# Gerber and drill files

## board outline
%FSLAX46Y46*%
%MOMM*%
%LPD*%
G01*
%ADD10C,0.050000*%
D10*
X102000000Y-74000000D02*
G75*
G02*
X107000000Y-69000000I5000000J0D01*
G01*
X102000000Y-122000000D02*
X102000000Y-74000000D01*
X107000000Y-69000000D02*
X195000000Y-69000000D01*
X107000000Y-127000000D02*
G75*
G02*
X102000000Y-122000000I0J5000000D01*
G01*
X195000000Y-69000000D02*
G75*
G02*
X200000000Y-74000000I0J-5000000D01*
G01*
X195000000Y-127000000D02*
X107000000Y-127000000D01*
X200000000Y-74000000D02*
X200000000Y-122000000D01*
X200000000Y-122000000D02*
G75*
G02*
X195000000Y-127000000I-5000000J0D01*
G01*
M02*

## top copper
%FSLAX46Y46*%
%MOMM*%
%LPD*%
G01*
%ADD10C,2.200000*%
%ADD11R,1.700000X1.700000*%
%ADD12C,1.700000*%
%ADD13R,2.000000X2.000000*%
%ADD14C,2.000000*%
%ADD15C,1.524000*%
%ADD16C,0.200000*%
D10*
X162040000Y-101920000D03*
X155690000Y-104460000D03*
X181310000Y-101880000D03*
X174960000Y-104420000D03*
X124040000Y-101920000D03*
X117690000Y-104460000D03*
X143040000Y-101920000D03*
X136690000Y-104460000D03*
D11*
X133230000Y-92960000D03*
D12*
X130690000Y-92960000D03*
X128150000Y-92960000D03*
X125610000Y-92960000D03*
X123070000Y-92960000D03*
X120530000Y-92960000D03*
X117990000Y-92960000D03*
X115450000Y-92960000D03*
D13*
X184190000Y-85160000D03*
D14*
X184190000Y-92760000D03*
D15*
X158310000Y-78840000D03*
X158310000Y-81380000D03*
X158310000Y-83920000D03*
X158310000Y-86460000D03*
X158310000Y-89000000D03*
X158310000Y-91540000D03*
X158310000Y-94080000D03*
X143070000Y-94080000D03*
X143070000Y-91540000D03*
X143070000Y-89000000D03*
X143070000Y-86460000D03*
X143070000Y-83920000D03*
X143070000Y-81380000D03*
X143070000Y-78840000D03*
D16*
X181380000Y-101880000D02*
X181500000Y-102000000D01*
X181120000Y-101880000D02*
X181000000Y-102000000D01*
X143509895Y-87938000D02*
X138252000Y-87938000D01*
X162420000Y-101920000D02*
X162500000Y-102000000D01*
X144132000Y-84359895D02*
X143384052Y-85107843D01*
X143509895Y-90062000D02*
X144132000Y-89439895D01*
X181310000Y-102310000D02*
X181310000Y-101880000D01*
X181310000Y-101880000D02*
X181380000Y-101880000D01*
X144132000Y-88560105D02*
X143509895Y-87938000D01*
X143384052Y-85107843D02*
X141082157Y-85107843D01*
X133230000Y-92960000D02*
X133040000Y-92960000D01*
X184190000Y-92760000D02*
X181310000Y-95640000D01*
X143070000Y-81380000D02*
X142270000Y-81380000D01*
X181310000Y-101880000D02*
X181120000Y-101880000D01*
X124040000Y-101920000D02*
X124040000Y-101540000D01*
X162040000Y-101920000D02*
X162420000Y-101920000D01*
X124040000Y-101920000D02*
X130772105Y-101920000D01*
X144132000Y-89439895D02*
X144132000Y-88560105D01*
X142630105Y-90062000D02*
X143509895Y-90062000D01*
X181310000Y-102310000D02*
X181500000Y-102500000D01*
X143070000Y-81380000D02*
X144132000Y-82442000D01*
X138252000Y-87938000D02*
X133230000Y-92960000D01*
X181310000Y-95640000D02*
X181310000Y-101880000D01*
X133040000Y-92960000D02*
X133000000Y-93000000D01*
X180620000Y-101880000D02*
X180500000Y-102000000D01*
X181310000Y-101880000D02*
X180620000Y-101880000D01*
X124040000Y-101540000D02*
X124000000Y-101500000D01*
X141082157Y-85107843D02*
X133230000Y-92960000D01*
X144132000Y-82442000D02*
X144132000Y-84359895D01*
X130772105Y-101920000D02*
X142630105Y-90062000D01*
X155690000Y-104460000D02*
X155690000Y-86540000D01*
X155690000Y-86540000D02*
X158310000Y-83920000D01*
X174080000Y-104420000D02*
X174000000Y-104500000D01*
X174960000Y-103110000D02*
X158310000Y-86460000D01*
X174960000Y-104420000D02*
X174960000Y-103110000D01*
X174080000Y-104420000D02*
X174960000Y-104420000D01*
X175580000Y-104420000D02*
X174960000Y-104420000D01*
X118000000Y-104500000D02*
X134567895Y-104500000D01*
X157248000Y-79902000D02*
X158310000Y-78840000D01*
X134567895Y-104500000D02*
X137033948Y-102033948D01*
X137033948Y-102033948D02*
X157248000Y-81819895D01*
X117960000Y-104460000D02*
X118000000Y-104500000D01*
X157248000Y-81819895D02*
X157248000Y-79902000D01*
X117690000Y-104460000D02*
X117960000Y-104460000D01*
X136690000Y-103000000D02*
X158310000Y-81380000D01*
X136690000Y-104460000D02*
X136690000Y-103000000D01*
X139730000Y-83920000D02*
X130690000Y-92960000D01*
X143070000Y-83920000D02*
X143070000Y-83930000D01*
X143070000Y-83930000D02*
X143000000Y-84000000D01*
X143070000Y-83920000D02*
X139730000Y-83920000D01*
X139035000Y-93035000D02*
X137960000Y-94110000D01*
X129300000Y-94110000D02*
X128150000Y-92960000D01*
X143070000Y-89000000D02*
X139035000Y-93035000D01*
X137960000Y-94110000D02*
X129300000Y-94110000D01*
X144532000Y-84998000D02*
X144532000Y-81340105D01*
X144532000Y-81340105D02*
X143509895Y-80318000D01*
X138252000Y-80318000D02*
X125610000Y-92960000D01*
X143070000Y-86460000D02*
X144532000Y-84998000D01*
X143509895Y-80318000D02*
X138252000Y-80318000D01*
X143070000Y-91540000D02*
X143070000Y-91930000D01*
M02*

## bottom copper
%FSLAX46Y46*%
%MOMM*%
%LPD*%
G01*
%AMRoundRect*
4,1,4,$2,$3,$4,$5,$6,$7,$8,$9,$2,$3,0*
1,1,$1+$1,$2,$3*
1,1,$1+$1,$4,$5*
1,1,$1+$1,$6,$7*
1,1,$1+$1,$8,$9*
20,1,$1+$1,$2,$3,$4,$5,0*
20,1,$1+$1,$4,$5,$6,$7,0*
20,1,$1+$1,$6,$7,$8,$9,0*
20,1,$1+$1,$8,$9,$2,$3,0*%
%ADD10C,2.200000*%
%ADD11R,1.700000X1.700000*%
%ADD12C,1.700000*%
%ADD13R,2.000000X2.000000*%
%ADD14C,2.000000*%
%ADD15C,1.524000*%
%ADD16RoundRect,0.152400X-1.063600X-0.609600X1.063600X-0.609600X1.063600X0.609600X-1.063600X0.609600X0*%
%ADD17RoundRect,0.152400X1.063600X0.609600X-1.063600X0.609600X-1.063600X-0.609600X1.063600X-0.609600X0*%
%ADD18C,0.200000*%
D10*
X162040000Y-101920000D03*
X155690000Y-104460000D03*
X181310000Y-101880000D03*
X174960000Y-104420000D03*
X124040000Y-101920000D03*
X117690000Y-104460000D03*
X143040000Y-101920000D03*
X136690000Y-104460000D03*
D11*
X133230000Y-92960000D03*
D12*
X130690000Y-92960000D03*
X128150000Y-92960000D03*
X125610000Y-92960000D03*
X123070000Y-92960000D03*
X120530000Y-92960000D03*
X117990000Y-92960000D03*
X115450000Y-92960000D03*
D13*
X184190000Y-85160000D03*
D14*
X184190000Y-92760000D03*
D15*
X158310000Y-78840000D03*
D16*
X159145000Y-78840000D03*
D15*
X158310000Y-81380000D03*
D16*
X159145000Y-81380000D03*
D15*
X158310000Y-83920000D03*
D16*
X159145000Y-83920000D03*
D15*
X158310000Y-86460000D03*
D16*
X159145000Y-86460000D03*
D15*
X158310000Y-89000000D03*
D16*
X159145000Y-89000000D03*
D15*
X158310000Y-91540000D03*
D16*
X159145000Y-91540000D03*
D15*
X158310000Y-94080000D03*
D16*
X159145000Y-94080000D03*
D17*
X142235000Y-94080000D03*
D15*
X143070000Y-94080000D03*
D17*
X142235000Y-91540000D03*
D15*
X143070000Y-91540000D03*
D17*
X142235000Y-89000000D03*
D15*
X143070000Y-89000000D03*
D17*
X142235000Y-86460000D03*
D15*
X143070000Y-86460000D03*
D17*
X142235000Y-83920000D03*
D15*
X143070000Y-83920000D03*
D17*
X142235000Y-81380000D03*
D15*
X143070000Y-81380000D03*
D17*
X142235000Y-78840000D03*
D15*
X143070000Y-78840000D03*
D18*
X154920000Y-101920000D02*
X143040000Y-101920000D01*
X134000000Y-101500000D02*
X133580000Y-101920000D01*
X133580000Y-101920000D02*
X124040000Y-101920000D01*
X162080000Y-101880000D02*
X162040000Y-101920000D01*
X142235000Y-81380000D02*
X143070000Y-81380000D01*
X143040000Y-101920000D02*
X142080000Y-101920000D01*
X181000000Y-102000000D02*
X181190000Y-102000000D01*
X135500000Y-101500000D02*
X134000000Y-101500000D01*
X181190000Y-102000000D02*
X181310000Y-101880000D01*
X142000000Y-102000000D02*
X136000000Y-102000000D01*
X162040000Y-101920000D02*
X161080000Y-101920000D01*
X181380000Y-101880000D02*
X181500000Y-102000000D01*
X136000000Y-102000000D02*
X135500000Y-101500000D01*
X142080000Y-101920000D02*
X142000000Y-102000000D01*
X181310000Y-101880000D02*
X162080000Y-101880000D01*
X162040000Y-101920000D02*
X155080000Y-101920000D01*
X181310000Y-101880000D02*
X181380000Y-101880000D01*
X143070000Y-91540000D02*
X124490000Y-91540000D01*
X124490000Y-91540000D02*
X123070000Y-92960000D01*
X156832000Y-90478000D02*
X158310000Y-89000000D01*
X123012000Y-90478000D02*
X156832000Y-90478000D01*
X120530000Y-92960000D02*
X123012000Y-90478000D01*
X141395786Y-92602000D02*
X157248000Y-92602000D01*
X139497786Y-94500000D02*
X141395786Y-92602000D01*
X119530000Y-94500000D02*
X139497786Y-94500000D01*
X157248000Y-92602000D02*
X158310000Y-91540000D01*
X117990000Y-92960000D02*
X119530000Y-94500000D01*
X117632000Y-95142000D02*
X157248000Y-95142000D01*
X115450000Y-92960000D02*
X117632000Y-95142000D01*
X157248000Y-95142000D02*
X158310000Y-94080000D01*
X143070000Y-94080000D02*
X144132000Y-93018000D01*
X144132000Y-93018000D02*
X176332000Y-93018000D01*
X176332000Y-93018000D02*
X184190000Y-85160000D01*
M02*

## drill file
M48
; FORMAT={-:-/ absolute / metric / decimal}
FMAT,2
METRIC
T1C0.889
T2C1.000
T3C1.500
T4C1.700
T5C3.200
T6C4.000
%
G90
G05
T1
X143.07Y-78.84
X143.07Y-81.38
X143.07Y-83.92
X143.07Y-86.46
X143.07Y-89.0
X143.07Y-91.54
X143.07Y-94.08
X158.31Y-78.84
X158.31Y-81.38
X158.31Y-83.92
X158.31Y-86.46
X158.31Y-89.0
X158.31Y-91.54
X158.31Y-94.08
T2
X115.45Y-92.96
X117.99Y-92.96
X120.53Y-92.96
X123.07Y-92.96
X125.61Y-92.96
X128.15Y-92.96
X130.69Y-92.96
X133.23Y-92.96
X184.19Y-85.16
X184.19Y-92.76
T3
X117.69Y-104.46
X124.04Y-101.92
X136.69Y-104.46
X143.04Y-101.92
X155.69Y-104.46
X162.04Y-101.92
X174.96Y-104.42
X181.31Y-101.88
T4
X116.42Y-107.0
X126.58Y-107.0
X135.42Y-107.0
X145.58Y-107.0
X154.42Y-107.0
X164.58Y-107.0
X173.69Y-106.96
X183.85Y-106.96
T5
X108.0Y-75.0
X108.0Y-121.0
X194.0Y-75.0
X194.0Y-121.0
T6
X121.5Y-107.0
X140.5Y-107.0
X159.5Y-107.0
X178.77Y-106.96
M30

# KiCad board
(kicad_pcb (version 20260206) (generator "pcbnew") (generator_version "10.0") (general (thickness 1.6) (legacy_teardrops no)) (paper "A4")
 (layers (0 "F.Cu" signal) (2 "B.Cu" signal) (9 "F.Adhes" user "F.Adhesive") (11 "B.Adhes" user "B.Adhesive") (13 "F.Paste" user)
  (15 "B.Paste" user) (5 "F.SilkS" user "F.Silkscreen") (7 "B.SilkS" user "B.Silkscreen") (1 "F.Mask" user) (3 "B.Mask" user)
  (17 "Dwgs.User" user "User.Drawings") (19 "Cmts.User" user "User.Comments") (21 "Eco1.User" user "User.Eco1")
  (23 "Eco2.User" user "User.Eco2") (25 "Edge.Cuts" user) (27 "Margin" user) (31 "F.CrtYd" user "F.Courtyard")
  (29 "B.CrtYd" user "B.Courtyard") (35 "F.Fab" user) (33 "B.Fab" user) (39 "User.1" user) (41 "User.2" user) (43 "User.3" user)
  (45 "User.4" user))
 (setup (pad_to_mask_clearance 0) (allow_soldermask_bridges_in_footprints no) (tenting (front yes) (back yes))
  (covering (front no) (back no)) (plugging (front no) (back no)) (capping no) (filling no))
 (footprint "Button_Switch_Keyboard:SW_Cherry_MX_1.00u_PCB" (layer "F.Cu") (at 162.04 101.92)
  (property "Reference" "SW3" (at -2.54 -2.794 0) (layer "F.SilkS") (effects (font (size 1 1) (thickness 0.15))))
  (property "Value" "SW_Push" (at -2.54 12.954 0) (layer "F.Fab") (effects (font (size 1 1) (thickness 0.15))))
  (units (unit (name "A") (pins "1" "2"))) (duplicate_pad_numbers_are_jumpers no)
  (pad "" np_thru_hole circle (at -7.62 5.08) (size 1.7 1.7) (drill 1.7) (layers "*.Cu" "*.Mask"))
  (pad "" np_thru_hole circle (at -2.54 5.08) (size 4 4) (drill 4) (layers "*.Cu" "*.Mask"))
  (pad "" np_thru_hole circle (at 2.54 5.08) (size 1.7 1.7) (drill 1.7) (layers "*.Cu" "*.Mask"))
  (pad "1" thru_hole circle (at 0 0) (size 2.2 2.2) (drill 1.5) (layers "*.Cu" "*.Mask") (remove_unused_layers no) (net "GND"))
  (pad "2" thru_hole circle (at -6.35 2.54) (size 2.2 2.2) (drill 1.5) (layers "*.Cu" "*.Mask") (remove_unused_layers no)
   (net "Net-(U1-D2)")))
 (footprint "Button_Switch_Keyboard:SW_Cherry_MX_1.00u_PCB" (layer "F.Cu") (at 181.31 101.88)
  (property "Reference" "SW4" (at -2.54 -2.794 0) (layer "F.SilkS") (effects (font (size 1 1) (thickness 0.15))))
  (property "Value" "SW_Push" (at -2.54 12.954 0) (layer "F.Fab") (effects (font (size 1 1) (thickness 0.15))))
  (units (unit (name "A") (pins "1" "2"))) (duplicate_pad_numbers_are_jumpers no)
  (pad "" np_thru_hole circle (at -7.62 5.08) (size 1.7 1.7) (drill 1.7) (layers "*.Cu" "*.Mask"))
  (pad "" np_thru_hole circle (at -2.54 5.08) (size 4 4) (drill 4) (layers "*.Cu" "*.Mask"))
  (pad "" np_thru_hole circle (at 2.54 5.08) (size 1.7 1.7) (drill 1.7) (layers "*.Cu" "*.Mask"))
  (pad "1" thru_hole circle (at 0 0) (size 2.2 2.2) (drill 1.5) (layers "*.Cu" "*.Mask") (remove_unused_layers no) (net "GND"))
  (pad "2" thru_hole circle (at -6.35 2.54) (size 2.2 2.2) (drill 1.5) (layers "*.Cu" "*.Mask") (remove_unused_layers no)
   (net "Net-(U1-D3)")))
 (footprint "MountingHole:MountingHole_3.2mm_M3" (layer "F.Cu") (at 194 121)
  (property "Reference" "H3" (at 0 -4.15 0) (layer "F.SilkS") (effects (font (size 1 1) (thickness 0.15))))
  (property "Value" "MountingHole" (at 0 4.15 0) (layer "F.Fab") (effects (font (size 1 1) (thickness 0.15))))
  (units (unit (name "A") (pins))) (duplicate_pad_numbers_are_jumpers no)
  (pad "" np_thru_hole circle (at 0 0) (size 3.2 3.2) (drill 3.2) (layers "*.Cu" "*.Mask")))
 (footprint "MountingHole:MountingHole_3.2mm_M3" (layer "F.Cu") (at 108 121)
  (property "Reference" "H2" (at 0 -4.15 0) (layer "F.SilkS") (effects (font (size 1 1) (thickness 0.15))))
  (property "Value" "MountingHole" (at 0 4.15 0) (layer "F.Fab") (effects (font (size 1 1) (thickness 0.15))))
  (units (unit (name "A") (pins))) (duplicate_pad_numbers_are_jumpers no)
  (pad "" np_thru_hole circle (at 0 0) (size 3.2 3.2) (drill 3.2) (layers "*.Cu" "*.Mask")))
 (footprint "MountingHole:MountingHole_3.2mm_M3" (layer "F.Cu") (at 194 75)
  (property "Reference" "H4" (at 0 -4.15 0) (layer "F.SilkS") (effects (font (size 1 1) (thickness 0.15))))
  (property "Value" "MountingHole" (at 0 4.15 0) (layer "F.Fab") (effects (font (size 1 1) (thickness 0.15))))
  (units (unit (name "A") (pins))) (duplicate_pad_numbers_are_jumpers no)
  (pad "" np_thru_hole circle (at 0 0) (size 3.2 3.2) (drill 3.2) (layers "*.Cu" "*.Mask")))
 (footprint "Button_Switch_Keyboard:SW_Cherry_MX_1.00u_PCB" (layer "F.Cu") (at 124.04 101.92)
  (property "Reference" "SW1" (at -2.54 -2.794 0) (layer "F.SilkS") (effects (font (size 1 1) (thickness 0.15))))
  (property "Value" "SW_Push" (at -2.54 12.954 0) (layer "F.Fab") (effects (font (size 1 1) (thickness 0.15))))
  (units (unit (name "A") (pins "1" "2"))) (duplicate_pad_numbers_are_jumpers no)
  (pad "" np_thru_hole circle (at -7.62 5.08) (size 1.7 1.7) (drill 1.7) (layers "*.Cu" "*.Mask"))
  (pad "" np_thru_hole circle (at -2.54 5.08) (size 4 4) (drill 4) (layers "*.Cu" "*.Mask"))
  (pad "" np_thru_hole circle (at 2.54 5.08) (size 1.7 1.7) (drill 1.7) (layers "*.Cu" "*.Mask"))
  (pad "1" thru_hole circle (at 0 0) (size 2.2 2.2) (drill 1.5) (layers "*.Cu" "*.Mask") (remove_unused_layers no) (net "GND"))
  (pad "2" thru_hole circle (at -6.35 2.54) (size 2.2 2.2) (drill 1.5) (layers "*.Cu" "*.Mask") (remove_unused_layers no)
   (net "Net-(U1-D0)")))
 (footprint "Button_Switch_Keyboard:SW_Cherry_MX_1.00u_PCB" (layer "F.Cu") (at 143.04 101.92)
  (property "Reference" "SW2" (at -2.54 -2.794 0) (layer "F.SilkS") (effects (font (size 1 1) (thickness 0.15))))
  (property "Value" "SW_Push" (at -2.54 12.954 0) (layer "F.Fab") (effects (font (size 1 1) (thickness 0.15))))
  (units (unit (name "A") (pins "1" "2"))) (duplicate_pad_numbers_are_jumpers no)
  (pad "" np_thru_hole circle (at -7.62 5.08) (size 1.7 1.7) (drill 1.7) (layers "*.Cu" "*.Mask"))
  (pad "" np_thru_hole circle (at -2.54 5.08) (size 4 4) (drill 4) (layers "*.Cu" "*.Mask"))
  (pad "" np_thru_hole circle (at 2.54 5.08) (size 1.7 1.7) (drill 1.7) (layers "*.Cu" "*.Mask"))
  (pad "1" thru_hole circle (at 0 0) (size 2.2 2.2) (drill 1.5) (layers "*.Cu" "*.Mask") (remove_unused_layers no) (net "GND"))
  (pad "2" thru_hole circle (at -6.35 2.54) (size 2.2 2.2) (drill 1.5) (layers "*.Cu" "*.Mask") (remove_unused_layers no)
   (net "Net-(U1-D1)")))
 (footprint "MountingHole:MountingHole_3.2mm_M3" (layer "F.Cu") (at 108 75)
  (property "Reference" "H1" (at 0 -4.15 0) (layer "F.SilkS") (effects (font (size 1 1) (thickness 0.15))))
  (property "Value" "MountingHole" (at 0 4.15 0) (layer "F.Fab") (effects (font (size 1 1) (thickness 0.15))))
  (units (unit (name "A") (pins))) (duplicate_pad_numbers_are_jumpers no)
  (pad "" np_thru_hole circle (at 0 0) (size 3.2 3.2) (drill 3.2) (layers "*.Cu" "*.Mask")))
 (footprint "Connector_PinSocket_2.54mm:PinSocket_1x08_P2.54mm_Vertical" (layer "B.Cu") (at 133.23 92.96 90)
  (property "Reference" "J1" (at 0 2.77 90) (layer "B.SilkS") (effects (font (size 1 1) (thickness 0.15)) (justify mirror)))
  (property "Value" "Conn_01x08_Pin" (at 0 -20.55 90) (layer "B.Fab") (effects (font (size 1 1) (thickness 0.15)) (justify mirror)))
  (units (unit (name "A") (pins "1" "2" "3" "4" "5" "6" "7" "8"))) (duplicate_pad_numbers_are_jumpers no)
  (pad "1" thru_hole rect (at 0 0 90) (size 1.7 1.7) (drill 1) (layers "*.Cu" "*.Mask") (remove_unused_layers no) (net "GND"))
  (pad "2" thru_hole circle (at 0 -2.54 90) (size 1.7 1.7) (drill 1) (layers "*.Cu" "*.Mask") (remove_unused_layers no) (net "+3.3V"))
  (pad "3" thru_hole circle (at 0 -5.08 90) (size 1.7 1.7) (drill 1) (layers "*.Cu" "*.Mask") (remove_unused_layers no) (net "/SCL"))
  (pad "4" thru_hole circle (at 0 -7.62 90) (size 1.7 1.7) (drill 1) (layers "*.Cu" "*.Mask") (remove_unused_layers no) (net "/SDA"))
  (pad "5" thru_hole circle (at 0 -10.16 90) (size 1.7 1.7) (drill 1) (layers "*.Cu" "*.Mask") (remove_unused_layers no) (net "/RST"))
  (pad "6" thru_hole circle (at 0 -12.7 90) (size 1.7 1.7) (drill 1) (layers "*.Cu" "*.Mask") (remove_unused_layers no) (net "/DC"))
  (pad "7" thru_hole circle (at 0 -15.24 90) (size 1.7 1.7) (drill 1) (layers "*.Cu" "*.Mask") (remove_unused_layers no) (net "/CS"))
  (pad "8" thru_hole circle (at 0 -17.78 90) (size 1.7 1.7) (drill 1) (layers "*.Cu" "*.Mask") (remove_unused_layers no) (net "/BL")))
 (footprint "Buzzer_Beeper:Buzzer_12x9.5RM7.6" (layer "B.Cu") (at 184.19 85.16 -90)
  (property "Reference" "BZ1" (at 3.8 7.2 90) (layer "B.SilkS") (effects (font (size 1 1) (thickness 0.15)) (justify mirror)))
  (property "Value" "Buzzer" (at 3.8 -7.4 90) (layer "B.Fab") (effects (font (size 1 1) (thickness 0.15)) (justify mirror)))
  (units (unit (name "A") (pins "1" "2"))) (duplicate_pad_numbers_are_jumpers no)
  (pad "1" thru_hole rect (at 0 0 270) (size 2 2) (drill 1) (layers "*.Cu" "*.Mask") (remove_unused_layers no) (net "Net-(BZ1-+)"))
  (pad "2" thru_hole circle (at 7.6 0 270) (size 2 2) (drill 1) (layers "*.Cu" "*.Mask") (remove_unused_layers no) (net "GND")))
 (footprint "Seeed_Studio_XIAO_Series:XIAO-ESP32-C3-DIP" (layer "B.Cu") (at 150.69 86.46 90)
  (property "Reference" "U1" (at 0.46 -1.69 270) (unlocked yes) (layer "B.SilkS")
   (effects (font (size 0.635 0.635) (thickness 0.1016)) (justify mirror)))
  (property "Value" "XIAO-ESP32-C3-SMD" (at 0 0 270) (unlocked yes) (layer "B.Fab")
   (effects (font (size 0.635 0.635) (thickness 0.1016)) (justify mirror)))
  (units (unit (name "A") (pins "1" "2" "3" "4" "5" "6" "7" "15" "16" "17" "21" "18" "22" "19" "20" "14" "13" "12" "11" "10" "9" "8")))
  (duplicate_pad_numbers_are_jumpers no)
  (pad "1" thru_hole circle (at 7.62 7.62) (size 1.524 1.524) (drill 0.889) (layers "*.Cu" "*.Mask") (remove_unused_layers no)
   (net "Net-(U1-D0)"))
  (pad "1" smd roundrect (at 7.62 8.455) (size 2.432 1.524) (layers "B.Cu" "B.Mask") (roundrect_rratio 0.1) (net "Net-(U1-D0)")
   (thermal_bridge_angle 45))
  (pad "2" thru_hole circle (at 5.08 7.62) (size 1.524 1.524) (drill 0.889) (layers "*.Cu" "*.Mask") (remove_unused_layers no)
   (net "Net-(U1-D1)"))
  (pad "2" smd roundrect (at 5.08 8.455) (size 2.432 1.524) (layers "B.Cu" "B.Mask") (roundrect_rratio 0.1) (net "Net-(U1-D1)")
   (thermal_bridge_angle 45))
  (pad "3" thru_hole circle (at 2.54 7.62) (size 1.524 1.524) (drill 0.889) (layers "*.Cu" "*.Mask") (remove_unused_layers no)
   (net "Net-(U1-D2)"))
  (pad "3" smd roundrect (at 2.54 8.455) (size 2.432 1.524) (layers "B.Cu" "B.Mask") (roundrect_rratio 0.1) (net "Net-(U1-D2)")
   (thermal_bridge_angle 45))
  (pad "4" thru_hole circle (at 0 7.62) (size 1.524 1.524) (drill 0.889) (layers "*.Cu" "*.Mask") (remove_unused_layers no)
   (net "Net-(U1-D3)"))
  (pad "4" smd roundrect (at 0 8.455) (size 2.432 1.524) (layers "B.Cu" "B.Mask") (roundrect_rratio 0.1) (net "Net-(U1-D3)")
   (thermal_bridge_angle 45))
  (pad "5" thru_hole circle (at -2.54 7.62) (size 1.524 1.524) (drill 0.889) (layers "*.Cu" "*.Mask") (remove_unused_layers no) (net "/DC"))
  (pad "5" smd roundrect (at -2.54 8.455) (size 2.432 1.524) (layers "B.Cu" "B.Mask") (roundrect_rratio 0.1) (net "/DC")
   (thermal_bridge_angle 45))
  (pad "6" thru_hole circle (at -5.08 7.62) (size 1.524 1.524) (drill 0.889) (layers "*.Cu" "*.Mask") (remove_unused_layers no) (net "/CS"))
  (pad "6" smd roundrect (at -5.08 8.455) (size 2.432 1.524) (layers "B.Cu" "B.Mask") (roundrect_rratio 0.1) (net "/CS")
   (thermal_bridge_angle 45))
  (pad "7" thru_hole circle (at -7.62 7.62) (size 1.524 1.524) (drill 0.889) (layers "*.Cu" "*.Mask") (remove_unused_layers no) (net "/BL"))
  (pad "7" smd roundrect (at -7.62 8.455) (size 2.432 1.524) (layers "B.Cu" "B.Mask") (roundrect_rratio 0.1) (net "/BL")
   (thermal_bridge_angle 45))
  (pad "8" smd roundrect (at -7.62 -8.455 180) (size 2.432 1.524) (layers "B.Cu" "B.Mask") (roundrect_rratio 0.1) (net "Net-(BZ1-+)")
   (thermal_bridge_angle 45))
  (pad "8" thru_hole circle (at -7.62 -7.62 180) (size 1.524 1.524) (drill 0.889) (layers "*.Cu" "*.Mask") (remove_unused_layers no)
   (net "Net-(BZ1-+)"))
  (pad "9" smd roundrect (at -5.08 -8.455 180) (size 2.432 1.524) (layers "B.Cu" "B.Mask") (roundrect_rratio 0.1) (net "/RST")
   (thermal_bridge_angle 45))
  (pad "9" thru_hole circle (at -5.08 -7.62 180) (size 1.524 1.524) (drill 0.889) (layers "*.Cu" "*.Mask") (remove_unused_layers no)
   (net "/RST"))
  (pad "10" smd roundrect (at -2.54 -8.455 180) (size 2.432 1.524) (layers "B.Cu" "B.Mask") (roundrect_rratio 0.1) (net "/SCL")
   (thermal_bridge_angle 45))
  (pad "10" thru_hole circle (at -2.54 -7.62 180) (size 1.524 1.524) (drill 0.889) (layers "*.Cu" "*.Mask") (remove_unused_layers no)
   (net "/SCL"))
  (pad "11" smd roundrect (at 0 -8.455 180) (size 2.432 1.524) (layers "B.Cu" "B.Mask") (roundrect_rratio 0.1) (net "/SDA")
   (thermal_bridge_angle 45))
  (pad "11" thru_hole circle (at 0 -7.62 180) (size 1.524 1.524) (drill 0.889) (layers "*.Cu" "*.Mask") (remove_unused_layers no)
   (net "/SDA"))
  (pad "12" smd roundrect (at 2.54 -8.455 180) (size 2.432 1.524) (layers "B.Cu" "B.Mask") (roundrect_rratio 0.1) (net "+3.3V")
   (thermal_bridge_angle 45))
  (pad "12" thru_hole circle (at 2.54 -7.62 180) (size 1.524 1.524) (drill 0.889) (layers "*.Cu" "*.Mask") (remove_unused_layers no)
   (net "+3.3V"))
  (pad "13" smd roundrect (at 5.08 -8.455 180) (size 2.432 1.524) (layers "B.Cu" "B.Mask") (roundrect_rratio 0.1) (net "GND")
   (thermal_bridge_angle 45))
  (pad "13" thru_hole circle (at 5.08 -7.62 180) (size 1.524 1.524) (drill 0.889) (layers "*.Cu" "*.Mask") (remove_unused_layers no)
   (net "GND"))
  (pad "14" smd roundrect (at 7.62 -8.455 180) (size 2.432 1.524) (layers "B.Cu" "B.Mask") (roundrect_rratio 0.1)
   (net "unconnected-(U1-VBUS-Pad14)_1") (thermal_bridge_angle 45))
  (pad "14" thru_hole circle (at 7.62 -7.62 180) (size 1.524 1.524) (drill 0.889) (layers "*.Cu" "*.Mask") (remove_unused_layers no)
   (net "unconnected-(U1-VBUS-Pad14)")))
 (gr_arc (start 102 74) (mid 103.464466 70.464466) (end 107 69) (stroke (width 0.05) (type default)) (layer "Edge.Cuts"))
 (gr_line (start 102 122) (end 102 74) (stroke (width 0.05) (type default)) (layer "Edge.Cuts"))
 (gr_line (start 107 69) (end 195 69) (stroke (width 0.05) (type default)) (layer "Edge.Cuts"))
 (gr_arc (start 107 127) (mid 103.464466 125.535534) (end 102 122) (stroke (width 0.05) (type default)) (layer "Edge.Cuts"))
 (gr_arc (start 195 69) (mid 198.535534 70.464466) (end 200 74) (stroke (width 0.05) (type default)) (layer "Edge.Cuts"))
 (gr_line (start 195 127) (end 107 127) (stroke (width 0.05) (type default)) (locked yes) (layer "Edge.Cuts"))
 (gr_line (start 200 74) (end 200 122) (stroke (width 0.05) (type default)) (layer "Edge.Cuts"))
 (gr_arc (start 200 122) (mid 198.535534 125.535534) (end 195 127) (stroke (width 0.05) (type default)) (layer "Edge.Cuts"))
 (segment (start 181.38 101.88) (end 181.5 102) (width 0.2) (layer "F.Cu") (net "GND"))
 (segment (start 181.12 101.88) (end 181 102) (width 0.2) (layer "F.Cu") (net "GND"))
 (segment (start 143.509895 87.938) (end 138.252 87.938) (width 0.2) (layer "F.Cu") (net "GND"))
 (segment (start 162.42 101.92) (end 162.5 102) (width 0.2) (layer "F.Cu") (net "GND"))
 (segment (start 144.132 84.359895) (end 143.384052 85.107843) (width 0.2) (layer "F.Cu") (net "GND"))
 (segment (start 143.509895 90.062) (end 144.132 89.439895) (width 0.2) (layer "F.Cu") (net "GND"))
 (segment (start 181.31 102.31) (end 181.31 101.88) (width 0.2) (layer "F.Cu") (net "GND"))
 (segment (start 181.31 101.88) (end 181.38 101.88) (width 0.2) (layer "F.Cu") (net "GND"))
 (segment (start 144.132 88.560105) (end 143.509895 87.938) (width 0.2) (layer "F.Cu") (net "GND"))
 (segment (start 143.384052 85.107843) (end 141.082157 85.107843) (width 0.2) (layer "F.Cu") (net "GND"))
 (segment (start 133.23 92.96) (end 133.04 92.96) (width 0.2) (layer "F.Cu") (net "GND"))
 (segment (start 184.19 92.76) (end 181.31 95.64) (width 0.2) (layer "F.Cu") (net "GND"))
 (segment (start 143.07 81.38) (end 142.27 81.38) (width 0.2) (layer "F.Cu") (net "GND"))
 (segment (start 181.31 101.88) (end 181.12 101.88) (width 0.2) (layer "F.Cu") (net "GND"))
 (segment (start 124.04 101.92) (end 124.04 101.54) (width 0.2) (layer "F.Cu") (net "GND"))
 (segment (start 162.04 101.92) (end 162.42 101.92) (width 0.2) (layer "F.Cu") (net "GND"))
 (segment (start 124.04 101.92) (end 130.772105 101.92) (width 0.2) (layer "F.Cu") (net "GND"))
 (segment (start 144.132 89.439895) (end 144.132 88.560105) (width 0.2) (layer "F.Cu") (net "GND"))
 (segment (start 142.630105 90.062) (end 143.509895 90.062) (width 0.2) (layer "F.Cu") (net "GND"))
 (segment (start 181.31 102.31) (end 181.5 102.5) (width 0.2) (layer "F.Cu") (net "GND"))
 (segment (start 143.07 81.38) (end 144.132 82.442) (width 0.2) (layer "F.Cu") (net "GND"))
 (segment (start 138.252 87.938) (end 133.23 92.96) (width 0.2) (layer "F.Cu") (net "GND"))
 (segment (start 181.31 95.64) (end 181.31 101.88) (width 0.2) (layer "F.Cu") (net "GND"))
 (segment (start 133.04 92.96) (end 133 93) (width 0.2) (layer "F.Cu") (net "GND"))
 (segment (start 180.62 101.88) (end 180.5 102) (width 0.2) (layer "F.Cu") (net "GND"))
 (segment (start 181.31 101.88) (end 180.62 101.88) (width 0.2) (layer "F.Cu") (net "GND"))
 (segment (start 124.04 101.54) (end 124 101.5) (width 0.2) (layer "F.Cu") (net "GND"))
 (segment (start 141.082157 85.107843) (end 133.23 92.96) (width 0.2) (layer "F.Cu") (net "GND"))
 (segment (start 144.132 82.442) (end 144.132 84.359895) (width 0.2) (layer "F.Cu") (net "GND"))
 (segment (start 130.772105 101.92) (end 142.630105 90.062) (width 0.2) (layer "F.Cu") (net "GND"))
 (segment (start 154.92 101.92) (end 143.04 101.92) (width 0.2) (layer "B.Cu") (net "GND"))
 (segment (start 134 101.5) (end 133.58 101.92) (width 0.2) (layer "B.Cu") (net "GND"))
 (segment (start 133.58 101.92) (end 124.04 101.92) (width 0.2) (layer "B.Cu") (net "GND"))
 (segment (start 162.08 101.88) (end 162.04 101.92) (width 0.2) (layer "B.Cu") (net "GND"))
 (segment (start 142.235 81.38) (end 143.07 81.38) (width 0.2) (layer "B.Cu") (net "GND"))
 (segment (start 143.04 101.92) (end 142.08 101.92) (width 0.2) (layer "B.Cu") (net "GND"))
 (segment (start 181 102) (end 181.19 102) (width 0.2) (layer "B.Cu") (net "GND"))
 (segment (start 135.5 101.5) (end 134 101.5) (width 0.2) (layer "B.Cu") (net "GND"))
 (segment (start 181.19 102) (end 181.31 101.88) (width 0.2) (layer "B.Cu") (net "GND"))
 (segment (start 142 102) (end 136 102) (width 0.2) (layer "B.Cu") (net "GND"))
 (segment (start 162.04 101.92) (end 161.08 101.92) (width 0.2) (layer "B.Cu") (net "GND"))
 (segment (start 181.38 101.88) (end 181.5 102) (width 0.2) (layer "B.Cu") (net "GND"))
 (segment (start 136 102) (end 135.5 101.5) (width 0.2) (layer "B.Cu") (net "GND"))
 (segment (start 142.08 101.92) (end 142 102) (width 0.2) (layer "B.Cu") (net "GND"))
 (segment (start 181.31 101.88) (end 162.08 101.88) (width 0.2) (layer "B.Cu") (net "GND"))
 (segment (start 162.04 101.92) (end 155.08 101.92) (width 0.2) (layer "B.Cu") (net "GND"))
 (segment (start 181.31 101.88) (end 181.38 101.88) (width 0.2) (layer "B.Cu") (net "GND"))
 (segment (start 155.69 104.46) (end 155.69 86.54) (width 0.2) (layer "F.Cu") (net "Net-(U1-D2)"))
 (segment (start 155.69 86.54) (end 158.31 83.92) (width 0.2) (layer "F.Cu") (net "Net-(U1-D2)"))
 (segment (start 174.08 104.42) (end 174 104.5) (width 0.2) (layer "F.Cu") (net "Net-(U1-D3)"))
 (segment (start 174.96 103.11) (end 158.31 86.46) (width 0.2) (layer "F.Cu") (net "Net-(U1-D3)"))
 (segment (start 174.96 104.42) (end 174.96 103.11) (width 0.2) (layer "F.Cu") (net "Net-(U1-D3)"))
 (segment (start 174.08 104.42) (end 174.96 104.42) (width 0.2) (layer "F.Cu") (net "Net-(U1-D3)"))
 (segment (start 175.58 104.42) (end 174.96 104.42) (width 0.2) (layer "F.Cu") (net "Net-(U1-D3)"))
 (segment (start 118 104.5) (end 134.567895 104.5) (width 0.2) (layer "F.Cu") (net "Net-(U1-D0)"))
 (segment (start 157.248 79.902) (end 158.31 78.84) (width 0.2) (layer "F.Cu") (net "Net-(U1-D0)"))
 (segment (start 134.567895 104.5) (end 137.033948 102.033948) (width 0.2) (layer "F.Cu") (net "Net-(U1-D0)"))
 (segment (start 137.033948 102.033948) (end 157.248 81.819895) (width 0.2) (layer "F.Cu") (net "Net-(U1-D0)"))
 (segment (start 117.96 104.46) (end 118 104.5) (width 0.2) (layer "F.Cu") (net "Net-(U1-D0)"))
 (segment (start 157.248 81.819895) (end 157.248 79.902) (width 0.2) (layer "F.Cu") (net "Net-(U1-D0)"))
 (segment (start 117.69 104.46) (end 117.96 104.46) (width 0.2) (layer "F.Cu") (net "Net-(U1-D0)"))
 (segment (start 136.69 103) (end 158.31 81.38) (width 0.2) (layer "F.Cu") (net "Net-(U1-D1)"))
 (segment (start 136.69 104.46) (end 136.69 103) (width 0.2) (layer "F.Cu") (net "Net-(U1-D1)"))
 (segment (start 139.73 83.92) (end 130.69 92.96) (width 0.2) (layer "F.Cu") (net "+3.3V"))
 (segment (start 143.07 83.92) (end 143.07 83.93) (width 0.2) (layer "F.Cu") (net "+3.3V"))
 (segment (start 143.07 83.93) (end 143 84) (width 0.2) (layer "F.Cu") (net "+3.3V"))
 (segment (start 143.07 83.92) (end 139.73 83.92) (width 0.2) (layer "F.Cu") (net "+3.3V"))
 (segment (start 139.035 93.035) (end 137.96 94.11) (width 0.2) (layer "F.Cu") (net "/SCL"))
 (segment (start 129.3 94.11) (end 128.15 92.96) (width 0.2) (layer "F.Cu") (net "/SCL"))
 (segment (start 143.07 89) (end 139.035 93.035) (width 0.2) (layer "F.Cu") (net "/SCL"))
 (segment (start 137.96 94.11) (end 129.3 94.11) (width 0.2) (layer "F.Cu") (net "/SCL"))
 (segment (start 144.532 84.998) (end 144.532 81.340105) (width 0.2) (layer "F.Cu") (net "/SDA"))
 (segment (start 144.532 81.340105) (end 143.509895 80.318) (width 0.2) (layer "F.Cu") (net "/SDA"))
 (segment (start 138.252 80.318) (end 125.61 92.96) (width 0.2) (layer "F.Cu") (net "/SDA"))
 (segment (start 143.07 86.46) (end 144.532 84.998) (width 0.2) (layer "F.Cu") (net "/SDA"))
 (segment (start 143.509895 80.318) (end 138.252 80.318) (width 0.2) (layer "F.Cu") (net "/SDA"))
 (segment (start 143.07 91.54) (end 143.07 91.93) (width 0.2) (layer "F.Cu") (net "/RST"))
 (segment (start 143.07 91.54) (end 124.49 91.54) (width 0.2) (layer "B.Cu") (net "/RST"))
 (segment (start 124.49 91.54) (end 123.07 92.96) (width 0.2) (layer "B.Cu") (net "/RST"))
 (segment (start 156.832 90.478) (end 158.31 89) (width 0.2) (layer "B.Cu") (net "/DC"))
 (segment (start 123.012 90.478) (end 156.832 90.478) (width 0.2) (layer "B.Cu") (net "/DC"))
 (segment (start 120.53 92.96) (end 123.012 90.478) (width 0.2) (layer "B.Cu") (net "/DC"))
 (segment (start 141.395786 92.602) (end 157.248 92.602) (width 0.2) (layer "B.Cu") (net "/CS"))
 (segment (start 139.497786 94.5) (end 141.395786 92.602) (width 0.2) (layer "B.Cu") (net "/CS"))
 (segment (start 119.53 94.5) (end 139.497786 94.5) (width 0.2) (layer "B.Cu") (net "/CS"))
 (segment (start 157.248 92.602) (end 158.31 91.54) (width 0.2) (layer "B.Cu") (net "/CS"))
 (segment (start 117.99 92.96) (end 119.53 94.5) (width 0.2) (layer "B.Cu") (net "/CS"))
 (segment (start 117.632 95.142) (end 157.248 95.142) (width 0.2) (layer "B.Cu") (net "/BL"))
 (segment (start 115.45 92.96) (end 117.632 95.142) (width 0.2) (layer "B.Cu") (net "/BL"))
 (segment (start 157.248 95.142) (end 158.31 94.08) (width 0.2) (layer "B.Cu") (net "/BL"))
 (segment (start 143.07 94.08) (end 144.132 93.018) (width 0.2) (layer "B.Cu") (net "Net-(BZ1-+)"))
 (segment (start 144.132 93.018) (end 176.332 93.018) (width 0.2) (layer "B.Cu") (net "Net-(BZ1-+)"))
 (segment (start 176.332 93.018) (end 184.19 85.16) (width 0.2) (layer "B.Cu") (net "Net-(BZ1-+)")))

